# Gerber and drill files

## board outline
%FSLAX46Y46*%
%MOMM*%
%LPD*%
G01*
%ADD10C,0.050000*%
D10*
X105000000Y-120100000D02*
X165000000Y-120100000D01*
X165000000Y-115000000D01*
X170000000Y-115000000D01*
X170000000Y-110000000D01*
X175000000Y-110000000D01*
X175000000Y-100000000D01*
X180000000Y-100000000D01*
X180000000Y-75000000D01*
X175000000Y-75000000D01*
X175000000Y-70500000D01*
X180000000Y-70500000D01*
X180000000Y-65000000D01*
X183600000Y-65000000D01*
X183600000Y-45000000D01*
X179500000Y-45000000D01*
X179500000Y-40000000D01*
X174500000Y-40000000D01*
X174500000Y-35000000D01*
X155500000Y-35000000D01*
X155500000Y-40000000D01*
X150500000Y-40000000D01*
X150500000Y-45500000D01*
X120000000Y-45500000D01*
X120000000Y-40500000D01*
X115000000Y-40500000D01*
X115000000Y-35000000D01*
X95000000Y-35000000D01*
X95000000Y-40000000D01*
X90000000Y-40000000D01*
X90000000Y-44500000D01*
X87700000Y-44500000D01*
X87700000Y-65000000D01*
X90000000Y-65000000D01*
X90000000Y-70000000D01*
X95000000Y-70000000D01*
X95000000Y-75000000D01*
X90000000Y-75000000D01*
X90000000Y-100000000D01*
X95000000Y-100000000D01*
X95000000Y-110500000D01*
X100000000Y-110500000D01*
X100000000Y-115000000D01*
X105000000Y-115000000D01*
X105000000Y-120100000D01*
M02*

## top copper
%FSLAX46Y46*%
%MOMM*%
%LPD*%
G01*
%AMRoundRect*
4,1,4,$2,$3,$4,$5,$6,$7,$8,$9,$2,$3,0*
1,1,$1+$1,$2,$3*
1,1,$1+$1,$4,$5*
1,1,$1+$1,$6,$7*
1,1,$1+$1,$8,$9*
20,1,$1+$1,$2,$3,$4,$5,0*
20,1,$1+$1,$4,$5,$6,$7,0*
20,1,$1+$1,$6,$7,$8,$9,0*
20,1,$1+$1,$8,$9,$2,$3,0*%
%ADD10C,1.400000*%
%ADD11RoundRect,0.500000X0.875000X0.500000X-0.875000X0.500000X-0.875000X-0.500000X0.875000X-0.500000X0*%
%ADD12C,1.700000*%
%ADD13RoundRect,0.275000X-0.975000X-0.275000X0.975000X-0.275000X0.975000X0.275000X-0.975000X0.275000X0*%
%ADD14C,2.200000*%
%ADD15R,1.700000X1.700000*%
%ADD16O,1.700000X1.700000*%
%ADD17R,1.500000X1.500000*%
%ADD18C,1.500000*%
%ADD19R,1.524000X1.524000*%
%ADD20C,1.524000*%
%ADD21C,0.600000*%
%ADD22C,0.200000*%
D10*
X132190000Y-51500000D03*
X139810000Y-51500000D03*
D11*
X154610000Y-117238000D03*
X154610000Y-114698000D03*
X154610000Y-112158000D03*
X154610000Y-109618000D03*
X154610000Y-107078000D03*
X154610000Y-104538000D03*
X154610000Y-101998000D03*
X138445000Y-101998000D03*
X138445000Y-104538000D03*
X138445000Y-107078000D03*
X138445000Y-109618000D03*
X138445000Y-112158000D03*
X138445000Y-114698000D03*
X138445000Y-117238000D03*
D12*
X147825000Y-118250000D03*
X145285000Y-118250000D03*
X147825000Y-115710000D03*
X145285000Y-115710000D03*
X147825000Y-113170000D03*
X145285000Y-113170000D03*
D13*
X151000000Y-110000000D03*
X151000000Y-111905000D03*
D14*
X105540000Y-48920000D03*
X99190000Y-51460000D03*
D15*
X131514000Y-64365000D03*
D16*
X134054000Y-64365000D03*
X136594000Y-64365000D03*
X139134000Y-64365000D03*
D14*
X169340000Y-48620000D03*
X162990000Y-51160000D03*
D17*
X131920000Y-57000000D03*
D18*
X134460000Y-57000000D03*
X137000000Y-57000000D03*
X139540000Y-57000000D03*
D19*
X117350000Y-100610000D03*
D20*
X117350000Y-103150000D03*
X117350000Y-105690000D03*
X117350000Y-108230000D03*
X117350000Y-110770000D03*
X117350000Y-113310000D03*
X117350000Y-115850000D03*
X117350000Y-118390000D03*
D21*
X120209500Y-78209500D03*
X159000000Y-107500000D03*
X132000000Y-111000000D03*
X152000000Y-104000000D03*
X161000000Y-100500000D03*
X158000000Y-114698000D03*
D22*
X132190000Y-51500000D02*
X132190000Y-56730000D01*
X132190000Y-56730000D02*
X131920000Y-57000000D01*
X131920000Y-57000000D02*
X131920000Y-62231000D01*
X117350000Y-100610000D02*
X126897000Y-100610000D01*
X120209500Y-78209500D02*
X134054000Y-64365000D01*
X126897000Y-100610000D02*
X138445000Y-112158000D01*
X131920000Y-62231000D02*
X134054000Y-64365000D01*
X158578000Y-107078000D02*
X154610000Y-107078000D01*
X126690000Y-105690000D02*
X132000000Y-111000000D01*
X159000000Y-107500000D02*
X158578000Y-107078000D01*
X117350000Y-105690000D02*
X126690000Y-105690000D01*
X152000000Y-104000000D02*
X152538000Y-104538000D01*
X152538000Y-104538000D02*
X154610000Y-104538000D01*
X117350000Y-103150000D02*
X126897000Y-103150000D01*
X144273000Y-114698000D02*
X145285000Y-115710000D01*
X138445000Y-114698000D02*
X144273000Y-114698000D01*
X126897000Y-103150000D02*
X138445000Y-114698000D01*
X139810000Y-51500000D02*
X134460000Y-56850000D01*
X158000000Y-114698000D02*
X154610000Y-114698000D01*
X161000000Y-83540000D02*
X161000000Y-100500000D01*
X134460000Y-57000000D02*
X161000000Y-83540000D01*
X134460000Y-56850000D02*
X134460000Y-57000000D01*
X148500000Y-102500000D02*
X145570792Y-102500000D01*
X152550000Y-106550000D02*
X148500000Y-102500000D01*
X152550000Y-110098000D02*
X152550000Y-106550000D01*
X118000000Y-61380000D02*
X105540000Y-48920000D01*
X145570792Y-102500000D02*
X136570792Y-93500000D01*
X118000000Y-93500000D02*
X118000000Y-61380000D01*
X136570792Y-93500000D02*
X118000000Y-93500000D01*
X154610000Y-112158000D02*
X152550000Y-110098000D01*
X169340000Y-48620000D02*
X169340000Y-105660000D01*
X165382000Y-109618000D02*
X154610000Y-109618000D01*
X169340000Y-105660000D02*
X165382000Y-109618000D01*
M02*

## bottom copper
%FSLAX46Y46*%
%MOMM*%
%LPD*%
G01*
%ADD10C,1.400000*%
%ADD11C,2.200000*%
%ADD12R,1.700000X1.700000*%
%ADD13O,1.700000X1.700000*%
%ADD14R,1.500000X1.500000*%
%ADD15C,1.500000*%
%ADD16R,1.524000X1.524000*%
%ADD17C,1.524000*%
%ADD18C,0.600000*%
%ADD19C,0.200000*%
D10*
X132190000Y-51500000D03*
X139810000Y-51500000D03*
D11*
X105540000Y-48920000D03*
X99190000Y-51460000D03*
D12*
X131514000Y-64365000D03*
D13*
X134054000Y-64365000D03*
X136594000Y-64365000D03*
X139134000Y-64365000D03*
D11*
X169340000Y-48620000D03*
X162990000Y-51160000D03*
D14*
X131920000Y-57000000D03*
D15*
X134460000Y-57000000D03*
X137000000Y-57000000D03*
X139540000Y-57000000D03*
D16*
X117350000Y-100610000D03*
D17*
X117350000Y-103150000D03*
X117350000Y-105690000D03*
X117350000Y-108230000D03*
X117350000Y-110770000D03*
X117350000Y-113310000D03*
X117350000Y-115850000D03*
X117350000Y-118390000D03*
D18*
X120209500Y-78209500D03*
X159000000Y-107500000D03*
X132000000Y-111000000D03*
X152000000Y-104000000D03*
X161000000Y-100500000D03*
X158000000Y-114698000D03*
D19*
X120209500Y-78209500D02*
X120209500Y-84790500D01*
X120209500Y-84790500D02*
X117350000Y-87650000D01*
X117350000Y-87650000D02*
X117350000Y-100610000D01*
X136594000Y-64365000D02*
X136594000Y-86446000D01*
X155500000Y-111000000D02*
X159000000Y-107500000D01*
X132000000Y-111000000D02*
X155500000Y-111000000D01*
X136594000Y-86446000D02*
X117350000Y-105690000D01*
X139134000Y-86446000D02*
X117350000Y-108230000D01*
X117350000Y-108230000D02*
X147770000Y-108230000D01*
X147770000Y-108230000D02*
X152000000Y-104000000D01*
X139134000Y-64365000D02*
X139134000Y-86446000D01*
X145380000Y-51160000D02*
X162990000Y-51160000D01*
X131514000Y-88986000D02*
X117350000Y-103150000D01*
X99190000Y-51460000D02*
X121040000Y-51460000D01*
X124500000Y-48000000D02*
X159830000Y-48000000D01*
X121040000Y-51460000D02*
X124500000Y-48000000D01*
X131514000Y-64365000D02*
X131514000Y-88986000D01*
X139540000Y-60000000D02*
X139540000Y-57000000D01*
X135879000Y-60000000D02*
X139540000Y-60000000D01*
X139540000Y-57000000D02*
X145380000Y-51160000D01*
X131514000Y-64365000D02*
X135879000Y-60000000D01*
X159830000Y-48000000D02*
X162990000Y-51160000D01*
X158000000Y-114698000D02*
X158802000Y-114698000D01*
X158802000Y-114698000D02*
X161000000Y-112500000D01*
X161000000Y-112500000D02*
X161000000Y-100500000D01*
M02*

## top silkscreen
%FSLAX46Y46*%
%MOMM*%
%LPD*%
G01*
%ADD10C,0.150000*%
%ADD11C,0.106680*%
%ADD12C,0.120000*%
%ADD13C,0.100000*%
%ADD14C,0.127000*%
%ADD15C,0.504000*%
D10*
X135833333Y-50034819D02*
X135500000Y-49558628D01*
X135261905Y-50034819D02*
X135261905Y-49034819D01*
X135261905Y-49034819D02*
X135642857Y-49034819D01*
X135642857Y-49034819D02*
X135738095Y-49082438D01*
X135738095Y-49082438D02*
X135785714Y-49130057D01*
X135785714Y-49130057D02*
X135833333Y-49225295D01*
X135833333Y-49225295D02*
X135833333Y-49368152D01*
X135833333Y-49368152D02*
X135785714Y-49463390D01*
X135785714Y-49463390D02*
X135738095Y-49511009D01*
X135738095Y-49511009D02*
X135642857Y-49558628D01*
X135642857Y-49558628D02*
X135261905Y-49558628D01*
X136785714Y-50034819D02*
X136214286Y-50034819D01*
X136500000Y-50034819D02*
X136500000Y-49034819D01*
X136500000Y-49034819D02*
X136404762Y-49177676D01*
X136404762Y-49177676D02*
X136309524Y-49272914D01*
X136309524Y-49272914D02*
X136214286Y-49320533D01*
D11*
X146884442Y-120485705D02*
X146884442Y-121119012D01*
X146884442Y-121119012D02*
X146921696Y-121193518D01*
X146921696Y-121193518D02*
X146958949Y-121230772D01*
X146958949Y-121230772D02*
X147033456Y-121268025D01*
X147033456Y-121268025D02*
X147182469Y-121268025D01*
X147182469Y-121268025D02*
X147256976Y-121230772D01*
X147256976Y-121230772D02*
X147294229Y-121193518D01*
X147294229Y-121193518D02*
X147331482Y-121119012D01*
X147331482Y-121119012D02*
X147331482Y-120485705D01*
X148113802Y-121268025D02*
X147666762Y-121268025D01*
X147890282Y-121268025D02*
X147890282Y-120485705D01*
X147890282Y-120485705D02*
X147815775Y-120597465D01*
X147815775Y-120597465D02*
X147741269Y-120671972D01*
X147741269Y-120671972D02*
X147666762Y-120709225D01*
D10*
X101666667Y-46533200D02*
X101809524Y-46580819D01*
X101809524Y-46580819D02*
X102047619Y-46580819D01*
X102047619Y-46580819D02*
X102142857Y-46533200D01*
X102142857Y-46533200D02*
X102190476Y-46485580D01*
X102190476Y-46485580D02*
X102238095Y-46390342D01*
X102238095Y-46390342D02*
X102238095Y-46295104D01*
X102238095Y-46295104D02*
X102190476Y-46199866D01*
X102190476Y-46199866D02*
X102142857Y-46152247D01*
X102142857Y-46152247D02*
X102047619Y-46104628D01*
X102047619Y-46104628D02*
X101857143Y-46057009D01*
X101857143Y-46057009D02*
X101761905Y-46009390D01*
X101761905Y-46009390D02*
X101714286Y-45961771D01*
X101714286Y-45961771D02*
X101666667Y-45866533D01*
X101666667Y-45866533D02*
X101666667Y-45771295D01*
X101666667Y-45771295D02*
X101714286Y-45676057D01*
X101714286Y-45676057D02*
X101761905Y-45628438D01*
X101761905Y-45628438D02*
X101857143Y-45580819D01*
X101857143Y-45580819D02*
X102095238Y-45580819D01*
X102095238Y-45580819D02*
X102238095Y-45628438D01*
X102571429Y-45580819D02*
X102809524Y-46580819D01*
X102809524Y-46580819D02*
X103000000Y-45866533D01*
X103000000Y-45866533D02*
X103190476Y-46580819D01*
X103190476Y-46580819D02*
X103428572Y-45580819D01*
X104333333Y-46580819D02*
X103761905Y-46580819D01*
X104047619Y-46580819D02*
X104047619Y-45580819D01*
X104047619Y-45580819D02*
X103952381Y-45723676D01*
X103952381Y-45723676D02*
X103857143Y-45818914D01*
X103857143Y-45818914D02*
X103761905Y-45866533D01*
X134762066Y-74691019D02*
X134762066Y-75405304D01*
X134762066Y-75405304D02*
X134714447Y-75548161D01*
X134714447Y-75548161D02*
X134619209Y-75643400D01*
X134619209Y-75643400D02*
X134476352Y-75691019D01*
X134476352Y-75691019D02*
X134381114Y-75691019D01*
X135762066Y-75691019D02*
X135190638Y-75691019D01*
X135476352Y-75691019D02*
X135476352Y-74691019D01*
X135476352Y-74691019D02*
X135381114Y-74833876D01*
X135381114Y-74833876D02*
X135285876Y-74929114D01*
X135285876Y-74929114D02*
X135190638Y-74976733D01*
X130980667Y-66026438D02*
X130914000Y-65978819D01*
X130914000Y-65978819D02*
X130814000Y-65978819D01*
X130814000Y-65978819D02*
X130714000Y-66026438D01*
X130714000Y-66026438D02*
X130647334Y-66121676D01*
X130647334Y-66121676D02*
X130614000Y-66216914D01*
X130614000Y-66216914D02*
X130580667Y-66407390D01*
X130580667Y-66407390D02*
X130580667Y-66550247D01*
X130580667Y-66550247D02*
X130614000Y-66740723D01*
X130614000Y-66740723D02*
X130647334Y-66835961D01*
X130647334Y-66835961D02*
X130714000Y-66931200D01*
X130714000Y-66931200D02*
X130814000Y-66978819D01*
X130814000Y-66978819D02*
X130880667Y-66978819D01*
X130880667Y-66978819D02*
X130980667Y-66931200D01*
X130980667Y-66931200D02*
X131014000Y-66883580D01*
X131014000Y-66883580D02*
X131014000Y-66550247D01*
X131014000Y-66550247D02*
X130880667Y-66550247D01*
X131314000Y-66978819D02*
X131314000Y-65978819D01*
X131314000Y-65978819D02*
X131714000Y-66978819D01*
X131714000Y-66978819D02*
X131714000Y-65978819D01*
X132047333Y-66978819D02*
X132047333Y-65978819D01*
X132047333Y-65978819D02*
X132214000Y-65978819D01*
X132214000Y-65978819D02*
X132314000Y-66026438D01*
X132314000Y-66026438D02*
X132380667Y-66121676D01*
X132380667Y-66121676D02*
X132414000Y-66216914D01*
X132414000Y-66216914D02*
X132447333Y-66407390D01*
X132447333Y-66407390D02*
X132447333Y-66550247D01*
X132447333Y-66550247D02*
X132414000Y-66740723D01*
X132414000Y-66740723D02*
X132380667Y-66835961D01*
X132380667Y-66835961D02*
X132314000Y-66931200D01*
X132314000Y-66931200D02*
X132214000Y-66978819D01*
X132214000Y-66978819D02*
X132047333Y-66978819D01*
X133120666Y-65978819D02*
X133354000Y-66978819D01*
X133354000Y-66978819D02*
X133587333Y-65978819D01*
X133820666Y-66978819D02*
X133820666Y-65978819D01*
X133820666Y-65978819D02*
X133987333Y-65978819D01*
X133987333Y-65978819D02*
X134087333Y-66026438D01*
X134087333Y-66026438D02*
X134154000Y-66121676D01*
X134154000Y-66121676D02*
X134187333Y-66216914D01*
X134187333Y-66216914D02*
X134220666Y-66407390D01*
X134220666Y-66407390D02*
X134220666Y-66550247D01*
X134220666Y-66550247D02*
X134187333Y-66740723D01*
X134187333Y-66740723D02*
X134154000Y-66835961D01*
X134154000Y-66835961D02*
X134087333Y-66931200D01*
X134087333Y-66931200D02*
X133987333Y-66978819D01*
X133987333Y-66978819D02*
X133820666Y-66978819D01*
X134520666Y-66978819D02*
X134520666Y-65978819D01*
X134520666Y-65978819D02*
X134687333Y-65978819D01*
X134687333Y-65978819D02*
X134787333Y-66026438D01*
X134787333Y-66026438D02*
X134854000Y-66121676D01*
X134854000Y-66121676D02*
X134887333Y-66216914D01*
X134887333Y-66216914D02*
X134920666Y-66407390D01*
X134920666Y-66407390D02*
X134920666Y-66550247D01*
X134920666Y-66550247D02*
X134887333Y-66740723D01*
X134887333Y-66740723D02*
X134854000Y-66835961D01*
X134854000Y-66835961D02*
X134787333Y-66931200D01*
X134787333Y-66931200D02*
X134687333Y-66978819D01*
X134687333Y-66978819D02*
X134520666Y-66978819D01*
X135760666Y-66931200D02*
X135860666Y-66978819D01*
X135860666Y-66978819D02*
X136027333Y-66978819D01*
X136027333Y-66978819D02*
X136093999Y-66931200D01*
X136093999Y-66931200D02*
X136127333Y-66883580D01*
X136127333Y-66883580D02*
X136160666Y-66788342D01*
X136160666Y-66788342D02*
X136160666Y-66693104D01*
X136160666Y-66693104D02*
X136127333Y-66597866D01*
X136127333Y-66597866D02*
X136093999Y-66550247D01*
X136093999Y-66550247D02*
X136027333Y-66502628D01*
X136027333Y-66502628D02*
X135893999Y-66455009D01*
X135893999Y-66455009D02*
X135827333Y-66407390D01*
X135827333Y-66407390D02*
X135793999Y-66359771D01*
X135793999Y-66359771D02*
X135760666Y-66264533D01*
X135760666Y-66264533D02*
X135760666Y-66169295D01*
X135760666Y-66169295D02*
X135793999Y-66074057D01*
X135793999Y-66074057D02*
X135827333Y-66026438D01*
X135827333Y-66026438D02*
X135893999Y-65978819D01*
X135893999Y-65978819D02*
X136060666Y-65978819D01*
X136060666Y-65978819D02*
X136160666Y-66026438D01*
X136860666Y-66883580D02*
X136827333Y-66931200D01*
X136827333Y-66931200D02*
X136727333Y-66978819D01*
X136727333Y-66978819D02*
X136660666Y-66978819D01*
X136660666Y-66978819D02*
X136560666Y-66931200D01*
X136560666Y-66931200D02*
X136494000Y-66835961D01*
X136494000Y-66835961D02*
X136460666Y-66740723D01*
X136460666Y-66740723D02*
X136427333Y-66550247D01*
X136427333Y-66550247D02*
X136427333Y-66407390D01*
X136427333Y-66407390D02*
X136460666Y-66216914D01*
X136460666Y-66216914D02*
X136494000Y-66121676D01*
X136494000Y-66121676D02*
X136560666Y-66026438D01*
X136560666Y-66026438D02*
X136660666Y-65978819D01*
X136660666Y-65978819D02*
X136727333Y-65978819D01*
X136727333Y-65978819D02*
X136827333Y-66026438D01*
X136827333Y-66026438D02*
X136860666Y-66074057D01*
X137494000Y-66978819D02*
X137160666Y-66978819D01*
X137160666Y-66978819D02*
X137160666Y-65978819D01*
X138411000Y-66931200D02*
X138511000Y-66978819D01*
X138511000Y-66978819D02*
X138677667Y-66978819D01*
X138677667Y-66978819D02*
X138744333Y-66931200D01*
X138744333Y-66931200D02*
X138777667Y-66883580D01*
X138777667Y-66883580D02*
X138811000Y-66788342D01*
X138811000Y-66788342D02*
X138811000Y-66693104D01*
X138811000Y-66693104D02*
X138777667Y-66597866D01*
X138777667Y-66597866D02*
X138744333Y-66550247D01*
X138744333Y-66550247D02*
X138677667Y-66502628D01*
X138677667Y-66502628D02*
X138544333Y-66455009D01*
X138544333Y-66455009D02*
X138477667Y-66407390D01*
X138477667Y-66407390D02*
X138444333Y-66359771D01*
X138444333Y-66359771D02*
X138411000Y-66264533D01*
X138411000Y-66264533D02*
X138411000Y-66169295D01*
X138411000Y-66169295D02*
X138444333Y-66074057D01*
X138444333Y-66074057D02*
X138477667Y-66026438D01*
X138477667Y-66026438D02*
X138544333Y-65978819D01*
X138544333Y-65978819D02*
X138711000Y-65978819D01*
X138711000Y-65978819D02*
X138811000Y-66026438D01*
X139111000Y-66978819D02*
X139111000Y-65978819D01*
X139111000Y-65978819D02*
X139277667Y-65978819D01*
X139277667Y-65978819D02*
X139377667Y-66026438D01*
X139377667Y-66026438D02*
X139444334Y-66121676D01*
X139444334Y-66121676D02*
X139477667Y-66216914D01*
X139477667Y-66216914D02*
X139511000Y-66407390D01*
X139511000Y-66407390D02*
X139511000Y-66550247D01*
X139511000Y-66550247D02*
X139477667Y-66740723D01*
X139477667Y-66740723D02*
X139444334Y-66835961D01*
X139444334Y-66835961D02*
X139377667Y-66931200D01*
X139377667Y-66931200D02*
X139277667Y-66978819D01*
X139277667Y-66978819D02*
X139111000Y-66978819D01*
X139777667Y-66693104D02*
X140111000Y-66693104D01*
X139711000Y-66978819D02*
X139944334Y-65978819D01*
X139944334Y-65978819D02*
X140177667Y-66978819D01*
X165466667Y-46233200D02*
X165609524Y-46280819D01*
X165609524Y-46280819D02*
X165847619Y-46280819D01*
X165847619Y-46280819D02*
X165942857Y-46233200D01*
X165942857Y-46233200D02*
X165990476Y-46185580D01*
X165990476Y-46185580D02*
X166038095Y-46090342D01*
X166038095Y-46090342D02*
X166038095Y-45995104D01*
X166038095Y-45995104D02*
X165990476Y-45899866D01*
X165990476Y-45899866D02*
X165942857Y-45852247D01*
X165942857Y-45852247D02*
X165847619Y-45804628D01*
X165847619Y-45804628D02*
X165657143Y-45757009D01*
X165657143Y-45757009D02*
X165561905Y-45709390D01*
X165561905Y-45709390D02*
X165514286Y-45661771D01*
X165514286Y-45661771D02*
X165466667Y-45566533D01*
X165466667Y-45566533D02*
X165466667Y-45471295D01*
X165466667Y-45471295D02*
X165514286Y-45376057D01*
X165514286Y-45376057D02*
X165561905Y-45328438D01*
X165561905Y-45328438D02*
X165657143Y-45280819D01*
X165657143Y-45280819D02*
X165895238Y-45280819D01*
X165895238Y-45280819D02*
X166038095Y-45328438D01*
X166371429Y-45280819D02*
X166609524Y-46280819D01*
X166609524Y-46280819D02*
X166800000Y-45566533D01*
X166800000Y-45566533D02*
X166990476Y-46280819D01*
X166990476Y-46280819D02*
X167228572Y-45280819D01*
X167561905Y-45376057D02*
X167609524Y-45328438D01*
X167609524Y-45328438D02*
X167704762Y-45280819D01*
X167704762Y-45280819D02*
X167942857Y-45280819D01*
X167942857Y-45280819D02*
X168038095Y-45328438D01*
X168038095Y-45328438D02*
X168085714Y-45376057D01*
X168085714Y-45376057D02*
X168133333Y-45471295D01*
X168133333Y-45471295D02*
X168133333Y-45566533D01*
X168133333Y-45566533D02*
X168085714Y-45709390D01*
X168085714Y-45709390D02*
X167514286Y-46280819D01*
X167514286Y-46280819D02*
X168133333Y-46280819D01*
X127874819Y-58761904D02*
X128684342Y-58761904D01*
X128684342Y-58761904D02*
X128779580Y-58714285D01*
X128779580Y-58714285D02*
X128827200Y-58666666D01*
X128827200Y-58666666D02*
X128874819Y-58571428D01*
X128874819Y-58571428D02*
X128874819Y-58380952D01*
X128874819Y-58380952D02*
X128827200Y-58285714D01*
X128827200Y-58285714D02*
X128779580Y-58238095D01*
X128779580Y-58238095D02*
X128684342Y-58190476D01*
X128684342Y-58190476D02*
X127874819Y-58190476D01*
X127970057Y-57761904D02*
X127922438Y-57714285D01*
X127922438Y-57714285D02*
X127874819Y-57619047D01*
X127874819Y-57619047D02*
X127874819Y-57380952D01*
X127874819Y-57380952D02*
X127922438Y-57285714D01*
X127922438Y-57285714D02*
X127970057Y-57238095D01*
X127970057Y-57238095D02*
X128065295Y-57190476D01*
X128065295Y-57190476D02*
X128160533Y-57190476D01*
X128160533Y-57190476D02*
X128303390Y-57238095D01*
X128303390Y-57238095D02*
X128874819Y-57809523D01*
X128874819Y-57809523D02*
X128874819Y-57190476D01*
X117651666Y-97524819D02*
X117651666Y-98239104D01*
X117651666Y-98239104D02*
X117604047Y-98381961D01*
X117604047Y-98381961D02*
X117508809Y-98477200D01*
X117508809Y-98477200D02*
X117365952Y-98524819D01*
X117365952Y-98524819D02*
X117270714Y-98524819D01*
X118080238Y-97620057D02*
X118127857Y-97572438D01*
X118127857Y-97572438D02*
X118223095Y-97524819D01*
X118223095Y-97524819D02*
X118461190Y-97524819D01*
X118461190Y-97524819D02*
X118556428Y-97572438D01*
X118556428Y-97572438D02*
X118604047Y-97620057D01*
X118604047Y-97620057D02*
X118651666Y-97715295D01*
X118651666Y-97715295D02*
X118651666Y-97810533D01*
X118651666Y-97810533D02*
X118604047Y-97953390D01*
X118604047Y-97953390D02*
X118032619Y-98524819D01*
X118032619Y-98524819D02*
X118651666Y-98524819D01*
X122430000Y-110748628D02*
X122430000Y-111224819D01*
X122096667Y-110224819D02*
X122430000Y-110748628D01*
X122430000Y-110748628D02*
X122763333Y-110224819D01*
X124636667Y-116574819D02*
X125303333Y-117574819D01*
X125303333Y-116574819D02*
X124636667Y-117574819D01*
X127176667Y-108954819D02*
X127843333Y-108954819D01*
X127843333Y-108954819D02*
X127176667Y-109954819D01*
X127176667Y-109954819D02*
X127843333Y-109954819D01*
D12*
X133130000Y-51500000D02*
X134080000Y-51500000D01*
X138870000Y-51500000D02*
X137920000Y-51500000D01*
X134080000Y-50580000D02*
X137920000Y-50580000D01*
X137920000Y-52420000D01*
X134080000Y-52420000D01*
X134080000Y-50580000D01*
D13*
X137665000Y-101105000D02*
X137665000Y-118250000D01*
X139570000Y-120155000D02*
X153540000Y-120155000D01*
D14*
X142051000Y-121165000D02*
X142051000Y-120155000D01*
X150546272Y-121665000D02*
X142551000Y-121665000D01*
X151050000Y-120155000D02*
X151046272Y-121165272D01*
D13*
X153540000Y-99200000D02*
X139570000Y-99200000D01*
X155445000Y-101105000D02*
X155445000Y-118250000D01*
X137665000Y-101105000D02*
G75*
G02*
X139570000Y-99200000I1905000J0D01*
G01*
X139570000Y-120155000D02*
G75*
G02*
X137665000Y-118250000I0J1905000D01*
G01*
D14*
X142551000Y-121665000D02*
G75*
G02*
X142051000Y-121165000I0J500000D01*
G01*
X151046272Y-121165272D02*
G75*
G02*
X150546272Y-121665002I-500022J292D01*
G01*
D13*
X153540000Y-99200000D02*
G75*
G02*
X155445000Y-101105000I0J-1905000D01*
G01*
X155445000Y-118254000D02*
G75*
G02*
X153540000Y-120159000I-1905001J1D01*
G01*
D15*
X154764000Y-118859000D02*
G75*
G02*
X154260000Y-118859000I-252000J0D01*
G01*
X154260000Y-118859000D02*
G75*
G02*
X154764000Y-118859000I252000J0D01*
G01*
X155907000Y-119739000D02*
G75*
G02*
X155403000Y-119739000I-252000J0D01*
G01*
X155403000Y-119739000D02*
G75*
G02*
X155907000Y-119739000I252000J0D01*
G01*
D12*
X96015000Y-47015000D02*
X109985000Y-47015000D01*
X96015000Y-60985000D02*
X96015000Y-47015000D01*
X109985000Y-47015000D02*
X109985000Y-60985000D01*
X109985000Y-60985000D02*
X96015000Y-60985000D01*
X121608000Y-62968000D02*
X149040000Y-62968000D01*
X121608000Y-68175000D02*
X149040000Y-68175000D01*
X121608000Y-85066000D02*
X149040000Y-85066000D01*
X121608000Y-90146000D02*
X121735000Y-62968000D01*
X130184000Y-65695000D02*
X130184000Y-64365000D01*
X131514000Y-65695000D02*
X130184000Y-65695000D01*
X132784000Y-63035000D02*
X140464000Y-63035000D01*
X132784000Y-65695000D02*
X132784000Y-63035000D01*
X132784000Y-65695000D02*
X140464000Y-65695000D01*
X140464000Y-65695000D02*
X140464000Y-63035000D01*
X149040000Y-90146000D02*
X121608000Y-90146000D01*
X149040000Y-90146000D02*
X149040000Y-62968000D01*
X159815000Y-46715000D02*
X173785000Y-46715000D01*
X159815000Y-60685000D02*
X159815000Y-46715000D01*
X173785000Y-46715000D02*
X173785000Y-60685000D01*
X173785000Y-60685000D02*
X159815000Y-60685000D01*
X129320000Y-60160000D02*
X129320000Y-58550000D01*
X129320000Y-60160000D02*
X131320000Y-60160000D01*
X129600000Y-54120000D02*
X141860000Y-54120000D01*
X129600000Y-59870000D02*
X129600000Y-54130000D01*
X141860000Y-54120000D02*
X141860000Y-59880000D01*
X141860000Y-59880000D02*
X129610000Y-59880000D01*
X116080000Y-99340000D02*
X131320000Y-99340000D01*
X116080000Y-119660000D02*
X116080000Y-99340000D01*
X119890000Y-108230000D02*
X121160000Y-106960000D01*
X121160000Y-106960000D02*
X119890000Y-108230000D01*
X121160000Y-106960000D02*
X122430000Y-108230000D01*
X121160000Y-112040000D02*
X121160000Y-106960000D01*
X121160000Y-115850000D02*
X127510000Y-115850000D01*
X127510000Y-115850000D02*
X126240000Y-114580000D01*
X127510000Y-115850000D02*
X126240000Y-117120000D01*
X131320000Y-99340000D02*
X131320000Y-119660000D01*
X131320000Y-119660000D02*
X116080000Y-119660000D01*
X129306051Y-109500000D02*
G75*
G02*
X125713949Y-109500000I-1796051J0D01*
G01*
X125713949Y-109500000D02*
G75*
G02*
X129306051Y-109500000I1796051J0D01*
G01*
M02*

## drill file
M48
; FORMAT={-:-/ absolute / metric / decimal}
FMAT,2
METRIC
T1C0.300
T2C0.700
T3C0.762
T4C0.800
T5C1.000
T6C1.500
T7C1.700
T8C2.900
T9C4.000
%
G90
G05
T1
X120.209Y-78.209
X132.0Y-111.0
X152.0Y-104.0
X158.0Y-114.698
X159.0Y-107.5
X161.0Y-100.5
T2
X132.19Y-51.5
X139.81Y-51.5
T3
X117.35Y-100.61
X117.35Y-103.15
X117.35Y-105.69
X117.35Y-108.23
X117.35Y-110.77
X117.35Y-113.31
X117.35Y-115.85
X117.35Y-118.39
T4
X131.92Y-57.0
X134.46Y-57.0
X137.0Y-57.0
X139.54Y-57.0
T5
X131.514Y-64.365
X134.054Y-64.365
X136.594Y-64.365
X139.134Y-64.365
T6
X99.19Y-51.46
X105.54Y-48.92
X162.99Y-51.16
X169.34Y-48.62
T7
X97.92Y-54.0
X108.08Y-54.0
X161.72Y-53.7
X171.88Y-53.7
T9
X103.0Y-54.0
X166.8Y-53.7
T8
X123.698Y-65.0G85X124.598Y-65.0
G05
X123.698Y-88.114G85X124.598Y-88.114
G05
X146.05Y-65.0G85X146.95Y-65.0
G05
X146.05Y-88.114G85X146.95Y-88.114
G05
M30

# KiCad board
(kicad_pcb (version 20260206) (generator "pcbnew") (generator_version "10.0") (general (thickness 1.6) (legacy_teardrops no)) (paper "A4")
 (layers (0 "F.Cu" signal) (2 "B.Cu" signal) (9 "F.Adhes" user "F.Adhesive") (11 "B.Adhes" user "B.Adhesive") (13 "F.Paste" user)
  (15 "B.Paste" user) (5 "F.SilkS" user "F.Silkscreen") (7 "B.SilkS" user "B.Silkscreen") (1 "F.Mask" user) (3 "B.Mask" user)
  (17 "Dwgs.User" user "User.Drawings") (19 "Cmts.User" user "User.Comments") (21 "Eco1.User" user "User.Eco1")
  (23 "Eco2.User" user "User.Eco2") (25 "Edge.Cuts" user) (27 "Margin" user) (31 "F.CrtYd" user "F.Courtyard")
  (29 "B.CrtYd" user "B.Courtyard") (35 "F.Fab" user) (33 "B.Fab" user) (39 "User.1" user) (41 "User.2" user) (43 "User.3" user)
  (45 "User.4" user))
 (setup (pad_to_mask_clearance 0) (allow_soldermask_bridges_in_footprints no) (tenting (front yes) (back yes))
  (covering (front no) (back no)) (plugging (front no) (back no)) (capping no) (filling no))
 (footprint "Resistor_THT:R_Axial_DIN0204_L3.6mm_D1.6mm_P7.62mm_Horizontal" (layer "F.Cu") (at 132.19 51.5)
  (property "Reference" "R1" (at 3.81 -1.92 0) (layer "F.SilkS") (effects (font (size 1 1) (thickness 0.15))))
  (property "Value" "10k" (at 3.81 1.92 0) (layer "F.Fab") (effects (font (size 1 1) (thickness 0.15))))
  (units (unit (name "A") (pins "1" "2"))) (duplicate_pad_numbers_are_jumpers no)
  (fp_line (start 0.94 0) (end 1.89 0) (stroke (width 0.12) (type solid)) (layer "F.SilkS"))
  (fp_line (start 6.68 0) (end 5.73 0) (stroke (width 0.12) (type solid)) (layer "F.SilkS"))
  (fp_rect (start 1.89 -0.92) (end 5.73 0.92) (stroke (width 0.12) (type solid)) (fill no) (layer "F.SilkS"))
  (pad "1" thru_hole circle (at 0 0) (size 1.4 1.4) (drill 0.7) (layers "*.Cu" "*.Mask") (remove_unused_layers no) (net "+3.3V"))
  (pad "2" thru_hole circle (at 7.62 0) (size 1.4 1.4) (drill 0.7) (layers "*.Cu" "*.Mask") (remove_unused_layers no) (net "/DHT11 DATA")))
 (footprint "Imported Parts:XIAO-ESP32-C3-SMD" (layer "F.Cu") (at 155.445 99.118 180)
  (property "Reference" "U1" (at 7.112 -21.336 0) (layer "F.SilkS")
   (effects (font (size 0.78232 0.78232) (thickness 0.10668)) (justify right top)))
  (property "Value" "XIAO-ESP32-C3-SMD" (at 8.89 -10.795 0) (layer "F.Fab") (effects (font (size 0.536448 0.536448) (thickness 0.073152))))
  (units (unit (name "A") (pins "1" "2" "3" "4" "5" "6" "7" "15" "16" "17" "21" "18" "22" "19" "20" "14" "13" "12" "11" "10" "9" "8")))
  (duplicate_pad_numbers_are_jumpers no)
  (fp_line (start 17.78 -1.987) (end 17.78 -19.132) (stroke (width 0.1) (type solid)) (layer "F.SilkS"))
  (fp_line (start 15.875 -21.037) (end 1.905 -21.037) (stroke (width 0.1) (type solid)) (layer "F.SilkS"))
  (fp_line (start 13.394 -22.047) (end 13.394 -21.037) (stroke (width 0.127) (type solid)) (layer "F.SilkS"))
  (fp_line (start 4.898728 -22.547) (end 12.894 -22.547) (stroke (width 0.127) (type solid)) (layer "F.SilkS"))
  (fp_line (start 4.395 -21.037) (end 4.398728 -22.047272) (stroke (width 0.127) (type solid)) (layer "F.SilkS"))
  (fp_line (start 1.905 -0.082) (end 15.875 -0.082) (stroke (width 0.1) (type solid)) (layer "F.SilkS"))
  (fp_line (start 0 -1.987) (end 0 -19.132) (stroke (width 0.1) (type solid)) (layer "F.SilkS"))
  (fp_arc (start 17.78 -1.987) (mid 17.222038 -0.639962) (end 15.875 -0.082) (stroke (width 0.1) (type solid)) (layer "F.SilkS"))
  (fp_arc (start 15.875 -21.037) (mid 17.222038 -20.479038) (end 17.78 -19.132) (stroke (width 0.1) (type solid)) (layer "F.SilkS"))
  (fp_arc (start 12.894 -22.547) (mid 13.247553 -22.400553) (end 13.394 -22.047) (stroke (width 0.127) (type default)) (layer "F.SilkS"))
  (fp_arc (start 4.398728 -22.047272) (mid 4.545272 -22.40064) (end 4.898728 -22.547) (stroke (width 0.127) (type default))
   (layer "F.SilkS"))
  (fp_arc (start 1.905 -0.082) (mid 0.557962 -0.639962) (end 0 -1.987) (stroke (width 0.1) (type solid)) (layer "F.SilkS"))
  (fp_arc (start 0 -19.136) (mid 0.557962 -20.483038) (end 1.905 -21.041) (stroke (width 0.1) (type solid)) (layer "F.SilkS"))
  (fp_circle (center 0.933 -19.741) (end 0.933 -19.995) (stroke (width 0.5) (type solid)) (fill yes) (layer "F.SilkS"))
  (fp_circle (center -0.21 -20.621) (end -0.21 -20.875) (stroke (width 0.5) (type solid)) (fill yes) (layer "F.SilkS"))
  (pad "1" smd roundrect (at 0.835 -18.12 180) (size 2.75 2) (layers "F.Cu" "F.Mask" "F.Paste") (roundrect_rratio 0.25)
   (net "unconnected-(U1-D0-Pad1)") (solder_mask_margin 0.0508) (thermal_bridge_angle 45))
  (pad "2" smd roundrect (at 0.835 -15.58 180) (size 2.75 2) (layers "F.Cu" "F.Mask" "F.Paste") (roundrect_rratio 0.25) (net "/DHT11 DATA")
   (solder_mask_margin 0.0508) (thermal_bridge_angle 45))
  (pad "3" smd roundrect (at 0.835 -13.04 180) (size 2.75 2) (layers "F.Cu" "F.Mask" "F.Paste") (roundrect_rratio 0.25) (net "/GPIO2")
   (solder_mask_margin 0.0508) (thermal_bridge_angle 45))
  (pad "4" smd roundrect (at 0.835 -10.5 180) (size 2.75 2) (layers "F.Cu" "F.Mask" "F.Paste") (roundrect_rratio 0.25) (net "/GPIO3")
   (solder_mask_margin 0.0508) (thermal_bridge_angle 45))
  (pad "5" smd roundrect (at 0.835 -7.96 180) (size 2.75 2) (layers "F.Cu" "F.Mask" "F.Paste") (roundrect_rratio 0.25) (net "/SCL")
   (solder_mask_margin 0.0508) (thermal_bridge_angle 45))
  (pad "6" smd roundrect (at 0.835 -5.42 180) (size 2.75 2) (layers "F.Cu" "F.Mask" "F.Paste") (roundrect_rratio 0.25) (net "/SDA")
   (solder_mask_margin 0.0508) (thermal_bridge_angle 45))
  (pad "7" smd roundrect (at 0.835 -2.88 180) (size 2.75 2) (layers "F.Cu" "F.Mask" "F.Paste") (roundrect_rratio 0.25)
   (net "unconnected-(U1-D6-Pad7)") (solder_mask_margin 0.0508) (thermal_bridge_angle 45))
  (pad "8" smd roundrect (at 17 -2.88 180) (size 2.75 2) (layers "F.Cu" "F.Mask" "F.Paste") (roundrect_rratio 0.25)
   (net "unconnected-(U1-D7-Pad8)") (solder_mask_margin 0.0508) (thermal_bridge_angle 45))
  (pad "9" smd roundrect (at 17 -5.42 180) (size 2.75 2) (layers "F.Cu" "F.Mask" "F.Paste") (roundrect_rratio 0.25)
   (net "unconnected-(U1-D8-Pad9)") (solder_mask_margin 0.0508) (thermal_bridge_angle 45))
  (pad "10" smd roundrect (at 17 -7.96 180) (size 2.75 2) (layers "F.Cu" "F.Mask" "F.Paste") (roundrect_rratio 0.25)
   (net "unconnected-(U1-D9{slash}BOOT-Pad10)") (solder_mask_margin 0.0508) (thermal_bridge_angle 45))
  (pad "11" smd roundrect (at 17 -10.5 180) (size 2.75 2) (layers "F.Cu" "F.Mask" "F.Paste") (roundrect_rratio 0.25)
   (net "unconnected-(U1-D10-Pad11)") (solder_mask_margin 0.0508) (thermal_bridge_angle 45))
  (pad "12" smd roundrect (at 17 -13.04 180) (size 2.75 2) (layers "F.Cu" "F.Mask" "F.Paste") (roundrect_rratio 0.25) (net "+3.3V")
   (solder_mask_margin 0.0508) (thermal_bridge_angle 45))
  (pad "13" smd roundrect (at 17 -15.58 180) (size 2.75 2) (layers "F.Cu" "F.Mask" "F.Paste") (roundrect_rratio 0.25) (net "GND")
   (solder_mask_margin 0.0508) (thermal_bridge_angle 45))
  (pad "14" smd roundrect (at 17 -18.12 180) (size 2.75 2) (layers "F.Cu" "F.Mask" "F.Paste") (roundrect_rratio 0.25) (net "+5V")
   (solder_mask_margin 0.0508) (thermal_bridge_angle 45))
  (pad "15" smd circle (at 7.62 -19.132 180) (size 1.7 1.7) (layers "F.Cu" "F.Mask" "F.Paste") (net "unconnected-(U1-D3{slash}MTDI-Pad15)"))
  (pad "16" smd circle (at 10.16 -19.132 180) (size 1.7 1.7) (layers "F.Cu" "F.Mask" "F.Paste") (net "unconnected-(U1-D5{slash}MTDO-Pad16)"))
  (pad "17" smd circle (at 7.62 -16.592 180) (size 1.7 1.7) (layers "F.Cu" "F.Mask" "F.Paste") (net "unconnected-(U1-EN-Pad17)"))
  (pad "18" smd circle (at 10.16 -16.592 180) (size 1.7 1.7) (layers "F.Cu" "F.Mask" "F.Paste") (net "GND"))
  (pad "19" smd circle (at 7.62 -14.052 180) (size 1.7 1.7) (layers "F.Cu" "F.Mask" "F.Paste") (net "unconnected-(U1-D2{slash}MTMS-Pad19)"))
  (pad "20" smd circle (at 10.16 -14.052 180) (size 1.7 1.7) (layers "F.Cu" "F.Mask" "F.Paste") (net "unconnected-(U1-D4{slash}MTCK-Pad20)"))
  (pad "21" smd roundrect (at 4.445 -10.882) (size 2.5 1.1) (layers "F.Cu" "F.Mask" "F.Paste") (roundrect_rratio 0.25)
   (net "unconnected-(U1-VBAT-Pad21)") (thermal_bridge_angle 45))
  (pad "22" smd roundrect (at 4.445 -12.787) (size 2.5 1.1) (layers "F.Cu" "F.Mask" "F.Paste") (roundrect_rratio 0.25)
   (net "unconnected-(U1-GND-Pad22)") (thermal_bridge_angle 45)))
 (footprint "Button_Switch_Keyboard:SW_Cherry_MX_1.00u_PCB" (layer "F.Cu") (at 105.54 48.92)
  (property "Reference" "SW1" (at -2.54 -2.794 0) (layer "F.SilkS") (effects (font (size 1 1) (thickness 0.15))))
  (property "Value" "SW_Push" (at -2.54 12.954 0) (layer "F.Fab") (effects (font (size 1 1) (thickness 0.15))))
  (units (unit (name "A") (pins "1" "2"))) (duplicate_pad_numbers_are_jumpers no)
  (fp_line (start -9.525 -1.905) (end 4.445 -1.905) (stroke (width 0.12) (type solid)) (layer "F.SilkS"))
  (fp_line (start -9.525 12.065) (end -9.525 -1.905) (stroke (width 0.12) (type solid)) (layer "F.SilkS"))
  (fp_line (start 4.445 -1.905) (end 4.445 12.065) (stroke (width 0.12) (type solid)) (layer "F.SilkS"))
  (fp_line (start 4.445 12.065) (end -9.525 12.065) (stroke (width 0.12) (type solid)) (layer "F.SilkS"))
  (pad "" np_thru_hole circle (at -7.62 5.08) (size 1.7 1.7) (drill 1.7) (layers "*.Cu" "*.Mask"))
  (pad "" np_thru_hole circle (at -2.54 5.08) (size 4 4) (drill 4) (layers "*.Cu" "*.Mask"))
  (pad "" np_thru_hole circle (at 2.54 5.08) (size 1.7 1.7) (drill 1.7) (layers "*.Cu" "*.Mask"))
  (pad "1" thru_hole circle (at 0 0) (size 2.2 2.2) (drill 1.5) (layers "*.Cu" "*.Mask") (remove_unused_layers no) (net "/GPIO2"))
  (pad "2" thru_hole circle (at -6.35 2.54) (size 2.2 2.2) (drill 1.5) (layers "*.Cu" "*.Mask") (remove_unused_layers no) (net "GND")))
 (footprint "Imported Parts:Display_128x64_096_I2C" (layer "F.Cu") (at 135.324 64.365)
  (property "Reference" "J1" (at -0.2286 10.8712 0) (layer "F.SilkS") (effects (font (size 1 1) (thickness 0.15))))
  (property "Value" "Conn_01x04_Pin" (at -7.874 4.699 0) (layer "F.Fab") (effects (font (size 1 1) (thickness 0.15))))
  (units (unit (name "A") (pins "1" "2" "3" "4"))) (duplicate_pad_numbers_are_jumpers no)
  (fp_line (start -13.716 -1.397) (end 13.716 -1.397) (stroke (width 0.12) (type solid)) (layer "F.SilkS"))
  (fp_line (start -13.716 3.81) (end 13.716 3.81) (stroke (width 0.12) (type solid)) (layer "F.SilkS"))
  (fp_line (start -13.716 20.701) (end 13.716 20.701) (stroke (width 0.12) (type solid)) (layer "F.SilkS"))
  (fp_line (start -13.716 25.781) (end -13.589 -1.397) (stroke (width 0.12) (type solid)) (layer "F.SilkS"))
  (fp_line (start -5.14 1.33) (end -5.14 0) (stroke (width 0.12) (type solid)) (layer "F.SilkS"))
  (fp_line (start -3.81 1.33) (end -5.14 1.33) (stroke (width 0.12) (type solid)) (layer "F.SilkS"))
  (fp_line (start -2.54 -1.33) (end 5.14 -1.33) (stroke (width 0.12) (type solid)) (layer "F.SilkS"))
  (fp_line (start -2.54 1.33) (end -2.54 -1.33) (stroke (width 0.12) (type solid)) (layer "F.SilkS"))
  (fp_line (start -2.54 1.33) (end 5.14 1.33) (stroke (width 0.12) (type solid)) (layer "F.SilkS"))
  (fp_line (start 5.14 1.33) (end 5.14 -1.33) (stroke (width 0.12) (type solid)) (layer "F.SilkS"))
  (fp_line (start 13.716 25.781) (end -13.716 25.781) (stroke (width 0.12) (type solid)) (layer "F.SilkS"))
  (fp_line (start 13.716 25.781) (end 13.716 -1.397) (stroke (width 0.12) (type solid)) (layer "F.SilkS"))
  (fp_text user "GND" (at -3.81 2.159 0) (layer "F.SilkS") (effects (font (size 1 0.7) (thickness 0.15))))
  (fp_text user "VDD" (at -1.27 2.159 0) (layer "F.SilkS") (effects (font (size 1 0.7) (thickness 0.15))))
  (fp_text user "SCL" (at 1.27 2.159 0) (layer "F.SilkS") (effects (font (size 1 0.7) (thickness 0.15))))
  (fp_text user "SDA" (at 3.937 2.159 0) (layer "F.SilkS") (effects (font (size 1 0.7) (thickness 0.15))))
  (pad "" np_thru_hole oval (at -11.176 0.635) (size 3.8 2.9) (drill oval 3.8 2.9) (layers "*.Cu" "*.Mask"))
  (pad "" np_thru_hole oval (at -11.176 23.749) (size 3.8 2.9) (drill oval 3.8 2.9) (layers "*.Cu" "*.Mask"))
  (pad "" np_thru_hole oval (at 11.176 0.635) (size 3.8 2.9) (drill oval 3.8 2.9) (layers "*.Cu" "*.Mask"))
  (pad "" np_thru_hole oval (at 11.176 23.749) (size 3.8 2.9) (drill oval 3.8 2.9) (layers "*.Cu" "*.Mask"))
  (pad "1" thru_hole rect (at -3.81 0 90) (size 1.7 1.7) (drill 1) (layers "*.Cu" "*.Mask") (remove_unused_layers no) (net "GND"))
  (pad "2" thru_hole oval (at -1.27 0 90) (size 1.7 1.7) (drill 1) (layers "*.Cu" "*.Mask") (remove_unused_layers no) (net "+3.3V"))
  (pad "3" thru_hole oval (at 1.27 0 90) (size 1.7 1.7) (drill 1) (layers "*.Cu" "*.Mask") (remove_unused_layers no) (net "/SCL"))
  (pad "4" thru_hole oval (at 3.81 0 90) (size 1.7 1.7) (drill 1) (layers "*.Cu" "*.Mask") (remove_unused_layers no) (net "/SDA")))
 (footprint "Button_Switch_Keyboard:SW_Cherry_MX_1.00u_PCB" (layer "F.Cu") (at 169.34 48.62)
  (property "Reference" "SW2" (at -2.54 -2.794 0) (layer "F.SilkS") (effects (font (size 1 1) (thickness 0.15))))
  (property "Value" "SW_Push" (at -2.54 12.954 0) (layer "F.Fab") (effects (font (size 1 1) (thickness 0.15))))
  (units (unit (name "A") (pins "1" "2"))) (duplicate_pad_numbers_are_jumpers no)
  (fp_line (start -9.525 -1.905) (end 4.445 -1.905) (stroke (width 0.12) (type solid)) (layer "F.SilkS"))
  (fp_line (start -9.525 12.065) (end -9.525 -1.905) (stroke (width 0.12) (type solid)) (layer "F.SilkS"))
  (fp_line (start 4.445 -1.905) (end 4.445 12.065) (stroke (width 0.12) (type solid)) (layer "F.SilkS"))
  (fp_line (start 4.445 12.065) (end -9.525 12.065) (stroke (width 0.12) (type solid)) (layer "F.SilkS"))
  (pad "" np_thru_hole circle (at -7.62 5.08) (size 1.7 1.7) (drill 1.7) (layers "*.Cu" "*.Mask"))
  (pad "" np_thru_hole circle (at -2.54 5.08) (size 4 4) (drill 4) (layers "*.Cu" "*.Mask"))
  (pad "" np_thru_hole circle (at 2.54 5.08) (size 1.7 1.7) (drill 1.7) (layers "*.Cu" "*.Mask"))
  (pad "1" thru_hole circle (at 0 0) (size 2.2 2.2) (drill 1.5) (layers "*.Cu" "*.Mask") (remove_unused_layers no) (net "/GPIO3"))
  (pad "2" thru_hole circle (at -6.35 2.54) (size 2.2 2.2) (drill 1.5) (layers "*.Cu" "*.Mask") (remove_unused_layers no) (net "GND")))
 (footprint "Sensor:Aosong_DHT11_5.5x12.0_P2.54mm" (layer "F.Cu") (at 131.92 57 90)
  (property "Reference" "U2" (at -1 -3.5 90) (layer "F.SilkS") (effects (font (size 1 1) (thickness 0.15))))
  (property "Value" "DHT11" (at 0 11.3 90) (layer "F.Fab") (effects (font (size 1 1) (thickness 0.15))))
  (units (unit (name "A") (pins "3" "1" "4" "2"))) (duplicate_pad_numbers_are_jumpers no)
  (fp_line (start -3.16 -2.6) (end -1.55 -2.6) (stroke (width 0.12) (type solid)) (layer "F.SilkS"))
  (fp_line (start -3.16 -2.6) (end -3.16 -0.6) (stroke (width 0.12) (type solid)) (layer "F.SilkS"))
  (fp_line (start 2.88 -2.32) (end 2.88 9.94) (stroke (width 0.12) (type solid)) (layer "F.SilkS"))
  (fp_line (start -2.87 -2.32) (end 2.87 -2.32) (stroke (width 0.12) (type solid)) (layer "F.SilkS"))
  (fp_line (start 2.88 9.94) (end -2.88 9.94) (stroke (width 0.12) (type solid)) (layer "F.SilkS"))
  (fp_line (start -2.88 9.94) (end -2.88 -2.31) (stroke (width 0.12) (type solid)) (layer "F.SilkS"))
  (pad "1" thru_hole rect (at 0 0 90) (size 1.5 1.5) (drill 0.8) (layers "*.Cu" "*.Mask") (remove_unused_layers no) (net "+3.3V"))
  (pad "2" thru_hole circle (at 0 2.54 90) (size 1.5 1.5) (drill 0.8) (layers "*.Cu" "*.Mask") (remove_unused_layers no) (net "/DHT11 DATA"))
  (pad "3" thru_hole circle (at 0 5.08 90) (size 1.5 1.5) (drill 0.8) (layers "*.Cu" "*.Mask") (remove_unused_layers no)
   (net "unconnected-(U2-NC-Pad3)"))
  (pad "4" thru_hole circle (at 0 7.62 90) (size 1.5 1.5) (drill 0.8) (layers "*.Cu" "*.Mask") (remove_unused_layers no) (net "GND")))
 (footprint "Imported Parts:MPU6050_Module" (layer "F.Cu") (at 117.35 100.61)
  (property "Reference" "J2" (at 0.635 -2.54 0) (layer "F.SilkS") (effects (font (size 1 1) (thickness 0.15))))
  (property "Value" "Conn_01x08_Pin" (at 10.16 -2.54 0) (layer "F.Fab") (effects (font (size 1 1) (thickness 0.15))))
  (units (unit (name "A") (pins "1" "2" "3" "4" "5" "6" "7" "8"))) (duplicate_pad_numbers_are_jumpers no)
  (fp_line (start -1.27 -1.27) (end 13.97 -1.27) (stroke (width 0.12) (type solid)) (layer "F.SilkS"))
  (fp_line (start -1.27 19.05) (end -1.27 -1.27) (stroke (width 0.12) (type solid)) (layer "F.SilkS"))
  (fp_line (start 2.54 7.62) (end 3.81 6.35) (stroke (width 0.12) (type solid)) (layer "F.SilkS"))
  (fp_line (start 3.81 6.35) (end 2.54 7.62) (stroke (width 0.12) (type solid)) (layer "F.SilkS"))
  (fp_line (start 3.81 6.35) (end 5.08 7.62) (stroke (width 0.12) (type solid)) (layer "F.SilkS"))
  (fp_line (start 3.81 11.43) (end 3.81 6.35) (stroke (width 0.12) (type solid)) (layer "F.SilkS"))
  (fp_line (start 3.81 15.24) (end 10.16 15.24) (stroke (width 0.12) (type solid)) (layer "F.SilkS"))
  (fp_line (start 10.16 15.24) (end 8.89 13.97) (stroke (width 0.12) (type solid)) (layer "F.SilkS"))
  (fp_line (start 10.16 15.24) (end 8.89 16.51) (stroke (width 0.12) (type solid)) (layer "F.SilkS"))
  (fp_line (start 13.97 -1.27) (end 13.97 19.05) (stroke (width 0.12) (type solid)) (layer "F.SilkS"))
  (fp_line (start 13.97 19.05) (end -1.27 19.05) (stroke (width 0.12) (type solid)) (layer "F.SilkS"))
  (fp_circle (center 10.16 8.89) (end 8.89 7.62) (stroke (width 0.12) (type solid)) (fill no) (layer "F.SilkS"))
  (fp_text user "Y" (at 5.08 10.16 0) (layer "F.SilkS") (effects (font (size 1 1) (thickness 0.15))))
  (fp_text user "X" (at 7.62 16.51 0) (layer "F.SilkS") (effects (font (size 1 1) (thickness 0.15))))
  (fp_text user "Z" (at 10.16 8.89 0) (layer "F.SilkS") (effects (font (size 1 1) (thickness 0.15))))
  (pad "1" thru_hole rect (at 0 0) (size 1.524 1.524) (drill 0.762) (layers "*.Cu" "*.Mask") (remove_unused_layers no) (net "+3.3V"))
  (pad "2" thru_hole circle (at 0 2.54) (size 1.524 1.524) (drill 0.762) (layers "*.Cu" "*.Mask") (remove_unused_layers no) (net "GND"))
  (pad "3" thru_hole circle (at 0 5.08) (size 1.524 1.524) (drill 0.762) (layers "*.Cu" "*.Mask") (remove_unused_layers no) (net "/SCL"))
  (pad "4" thru_hole circle (at 0 7.62) (size 1.524 1.524) (drill 0.762) (layers "*.Cu" "*.Mask") (remove_unused_layers no) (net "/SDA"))
  (pad "5" thru_hole circle (at 0 10.16) (size 1.524 1.524) (drill 0.762) (layers "*.Cu" "*.Mask") (remove_unused_layers no)
   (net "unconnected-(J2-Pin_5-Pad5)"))
  (pad "6" thru_hole circle (at 0 12.7) (size 1.524 1.524) (drill 0.762) (layers "*.Cu" "*.Mask") (remove_unused_layers no)
   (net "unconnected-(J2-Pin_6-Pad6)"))
  (pad "7" thru_hole circle (at 0 15.24) (size 1.524 1.524) (drill 0.762) (layers "*.Cu" "*.Mask") (remove_unused_layers no)
   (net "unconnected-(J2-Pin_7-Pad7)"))
  (pad "8" thru_hole circle (at 0 17.78) (size 1.524 1.524) (drill 0.762) (layers "*.Cu" "*.Mask") (remove_unused_layers no)
   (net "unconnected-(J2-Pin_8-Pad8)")))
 (gr_poly
  (pts (xy 105 120.1) (xy 165 120.1) (xy 165 115) (xy 170 115) (xy 170 110) (xy 175 110) (xy 175 100) (xy 180 100) (xy 180 75) (xy 175 75)
   (xy 175 70.5) (xy 180 70.5) (xy 180 65) (xy 183.6 65) (xy 183.6 45) (xy 179.5 45) (xy 179.5 40) (xy 174.5 40) (xy 174.5 35) (xy 155.5 35)
   (xy 155.5 40) (xy 150.5 40) (xy 150.5 45.5) (xy 120 45.5) (xy 120 40.5) (xy 115 40.5) (xy 115 35) (xy 95 35) (xy 95 40) (xy 90 40)
   (xy 90 44.5) (xy 87.7 44.5) (xy 87.7 65) (xy 90 65) (xy 90 70) (xy 95 70) (xy 95 75) (xy 90 75) (xy 90 100) (xy 95 100) (xy 95 110.5)
   (xy 100 110.5) (xy 100 115) (xy 105 115))
  (stroke (width 0.05) (type solid)) (fill no) (layer "Edge.Cuts"))
 (segment (start 132.19 51.5) (end 132.19 56.73) (width 0.2) (layer "F.Cu") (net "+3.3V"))
 (segment (start 132.19 56.73) (end 131.92 57) (width 0.2) (layer "F.Cu") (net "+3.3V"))
 (segment (start 131.92 57) (end 131.92 62.231) (width 0.2) (layer "F.Cu") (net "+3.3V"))
 (segment (start 117.35 100.61) (end 126.897 100.61) (width 0.2) (layer "F.Cu") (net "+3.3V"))
 (segment (start 120.2095 78.2095) (end 134.054 64.365) (width 0.2) (layer "F.Cu") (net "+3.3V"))
 (segment (start 126.897 100.61) (end 138.445 112.158) (width 0.2) (layer "F.Cu") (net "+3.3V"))
 (segment (start 131.92 62.231) (end 134.054 64.365) (width 0.2) (layer "F.Cu") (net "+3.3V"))
 (via (at 120.2095 78.2095) (size 0.6) (drill 0.3) (layers "F.Cu" "B.Cu") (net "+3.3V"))
 (segment (start 120.2095 78.2095) (end 120.2095 84.7905) (width 0.2) (layer "B.Cu") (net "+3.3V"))
 (segment (start 120.2095 84.7905) (end 117.35 87.65) (width 0.2) (layer "B.Cu") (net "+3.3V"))
 (segment (start 117.35 87.65) (end 117.35 100.61) (width 0.2) (layer "B.Cu") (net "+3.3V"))
 (segment (start 158.578 107.078) (end 154.61 107.078) (width 0.2) (layer "F.Cu") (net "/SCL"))
 (segment (start 126.69 105.69) (end 132 111) (width 0.2) (layer "F.Cu") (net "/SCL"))
 (segment (start 159 107.5) (end 158.578 107.078) (width 0.2) (layer "F.Cu") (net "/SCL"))
 (segment (start 117.35 105.69) (end 126.69 105.69) (width 0.2) (layer "F.Cu") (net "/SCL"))
 (via (at 159 107.5) (size 0.6) (drill 0.3) (layers "F.Cu" "B.Cu") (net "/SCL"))
 (via (at 132 111) (size 0.6) (drill 0.3) (layers "F.Cu" "B.Cu") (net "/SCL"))
 (segment (start 136.594 64.365) (end 136.594 86.446) (width 0.2) (layer "B.Cu") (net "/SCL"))
 (segment (start 155.5 111) (end 159 107.5) (width 0.2) (layer "B.Cu") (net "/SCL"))
 (segment (start 132 111) (end 155.5 111) (width 0.2) (layer "B.Cu") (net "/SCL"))
 (segment (start 136.594 86.446) (end 117.35 105.69) (width 0.2) (layer "B.Cu") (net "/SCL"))
 (segment (start 152 104) (end 152.538 104.538) (width 0.2) (layer "F.Cu") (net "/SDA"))
 (segment (start 152.538 104.538) (end 154.61 104.538) (width 0.2) (layer "F.Cu") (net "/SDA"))
 (via (at 152 104) (size 0.6) (drill 0.3) (layers "F.Cu" "B.Cu") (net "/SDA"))
 (segment (start 139.134 86.446) (end 117.35 108.23) (width 0.2) (layer "B.Cu") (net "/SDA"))
 (segment (start 117.35 108.23) (end 147.77 108.23) (width 0.2) (layer "B.Cu") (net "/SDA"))
 (segment (start 147.77 108.23) (end 152 104) (width 0.2) (layer "B.Cu") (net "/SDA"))
 (segment (start 139.134 64.365) (end 139.134 86.446) (width 0.2) (layer "B.Cu") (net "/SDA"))
 (segment (start 117.35 103.15) (end 126.897 103.15) (width 0.2) (layer "F.Cu") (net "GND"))
 (segment (start 144.273 114.698) (end 145.285 115.71) (width 0.2) (layer "F.Cu") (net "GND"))
 (segment (start 138.445 114.698) (end 144.273 114.698) (width 0.2) (layer "F.Cu") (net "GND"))
 (segment (start 126.897 103.15) (end 138.445 114.698) (width 0.2) (layer "F.Cu") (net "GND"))
 (segment (start 145.38 51.16) (end 162.99 51.16) (width 0.2) (layer "B.Cu") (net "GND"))
 (segment (start 131.514 88.986) (end 117.35 103.15) (width 0.2) (layer "B.Cu") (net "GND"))
 (segment (start 99.19 51.46) (end 121.04 51.46) (width 0.2) (layer "B.Cu") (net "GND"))
 (segment (start 124.5 48) (end 159.83 48) (width 0.2) (layer "B.Cu") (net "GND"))
 (segment (start 121.04 51.46) (end 124.5 48) (width 0.2) (layer "B.Cu") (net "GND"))
 (segment (start 131.514 64.365) (end 131.514 88.986) (width 0.2) (layer "B.Cu") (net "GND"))
 (segment (start 139.54 60) (end 139.54 57) (width 0.2) (layer "B.Cu") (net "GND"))
 (segment (start 135.879 60) (end 139.54 60) (width 0.2) (layer "B.Cu") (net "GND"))
 (segment (start 139.54 57) (end 145.38 51.16) (width 0.2) (layer "B.Cu") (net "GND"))
 (segment (start 131.514 64.365) (end 135.879 60) (width 0.2) (layer "B.Cu") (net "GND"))
 (segment (start 159.83 48) (end 162.99 51.16) (width 0.2) (layer "B.Cu") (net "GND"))
 (segment (start 139.81 51.5) (end 134.46 56.85) (width 0.2) (layer "F.Cu") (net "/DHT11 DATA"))
 (segment (start 158 114.698) (end 154.61 114.698) (width 0.2) (layer "F.Cu") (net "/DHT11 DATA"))
 (segment (start 161 83.54) (end 161 100.5) (width 0.2) (layer "F.Cu") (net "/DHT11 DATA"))
 (segment (start 134.46 57) (end 161 83.54) (width 0.2) (layer "F.Cu") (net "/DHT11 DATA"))
 (segment (start 134.46 56.85) (end 134.46 57) (width 0.2) (layer "F.Cu") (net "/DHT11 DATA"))
 (via (at 161 100.5) (size 0.6) (drill 0.3) (layers "F.Cu" "B.Cu") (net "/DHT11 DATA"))
 (via (at 158 114.698) (size 0.6) (drill 0.3) (layers "F.Cu" "B.Cu") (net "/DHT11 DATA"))
 (segment (start 158 114.698) (end 158.802 114.698) (width 0.2) (layer "B.Cu") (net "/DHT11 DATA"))
 (segment (start 158.802 114.698) (end 161 112.5) (width 0.2) (layer "B.Cu") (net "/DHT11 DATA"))
 (segment (start 161 112.5) (end 161 100.5) (width 0.2) (layer "B.Cu") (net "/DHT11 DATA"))
 (segment (start 148.5 102.5) (end 145.570792 102.5) (width 0.2) (layer "F.Cu") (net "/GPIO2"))
 (segment (start 152.55 106.55) (end 148.5 102.5) (width 0.2) (layer "F.Cu") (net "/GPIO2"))
 (segment (start 152.55 110.098) (end 152.55 106.55) (width 0.2) (layer "F.Cu") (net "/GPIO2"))
 (segment (start 118 61.38) (end 105.54 48.92) (width 0.2) (layer "F.Cu") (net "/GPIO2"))
 (segment (start 145.570792 102.5) (end 136.570792 93.5) (width 0.2) (layer "F.Cu") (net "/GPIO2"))
 (segment (start 118 93.5) (end 118 61.38) (width 0.2) (layer "F.Cu") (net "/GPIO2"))
 (segment (start 136.570792 93.5) (end 118 93.5) (width 0.2) (layer "F.Cu") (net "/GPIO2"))
 (segment (start 154.61 112.158) (end 152.55 110.098) (width 0.2) (layer "F.Cu") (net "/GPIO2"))
 (segment (start 169.34 48.62) (end 169.34 105.66) (width 0.2) (layer "F.Cu") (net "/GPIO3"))
 (segment (start 165.382 109.618) (end 154.61 109.618) (width 0.2) (layer "F.Cu") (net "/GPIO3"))
 (segment (start 169.34 105.66) (end 165.382 109.618) (width 0.2) (layer "F.Cu") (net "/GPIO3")))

